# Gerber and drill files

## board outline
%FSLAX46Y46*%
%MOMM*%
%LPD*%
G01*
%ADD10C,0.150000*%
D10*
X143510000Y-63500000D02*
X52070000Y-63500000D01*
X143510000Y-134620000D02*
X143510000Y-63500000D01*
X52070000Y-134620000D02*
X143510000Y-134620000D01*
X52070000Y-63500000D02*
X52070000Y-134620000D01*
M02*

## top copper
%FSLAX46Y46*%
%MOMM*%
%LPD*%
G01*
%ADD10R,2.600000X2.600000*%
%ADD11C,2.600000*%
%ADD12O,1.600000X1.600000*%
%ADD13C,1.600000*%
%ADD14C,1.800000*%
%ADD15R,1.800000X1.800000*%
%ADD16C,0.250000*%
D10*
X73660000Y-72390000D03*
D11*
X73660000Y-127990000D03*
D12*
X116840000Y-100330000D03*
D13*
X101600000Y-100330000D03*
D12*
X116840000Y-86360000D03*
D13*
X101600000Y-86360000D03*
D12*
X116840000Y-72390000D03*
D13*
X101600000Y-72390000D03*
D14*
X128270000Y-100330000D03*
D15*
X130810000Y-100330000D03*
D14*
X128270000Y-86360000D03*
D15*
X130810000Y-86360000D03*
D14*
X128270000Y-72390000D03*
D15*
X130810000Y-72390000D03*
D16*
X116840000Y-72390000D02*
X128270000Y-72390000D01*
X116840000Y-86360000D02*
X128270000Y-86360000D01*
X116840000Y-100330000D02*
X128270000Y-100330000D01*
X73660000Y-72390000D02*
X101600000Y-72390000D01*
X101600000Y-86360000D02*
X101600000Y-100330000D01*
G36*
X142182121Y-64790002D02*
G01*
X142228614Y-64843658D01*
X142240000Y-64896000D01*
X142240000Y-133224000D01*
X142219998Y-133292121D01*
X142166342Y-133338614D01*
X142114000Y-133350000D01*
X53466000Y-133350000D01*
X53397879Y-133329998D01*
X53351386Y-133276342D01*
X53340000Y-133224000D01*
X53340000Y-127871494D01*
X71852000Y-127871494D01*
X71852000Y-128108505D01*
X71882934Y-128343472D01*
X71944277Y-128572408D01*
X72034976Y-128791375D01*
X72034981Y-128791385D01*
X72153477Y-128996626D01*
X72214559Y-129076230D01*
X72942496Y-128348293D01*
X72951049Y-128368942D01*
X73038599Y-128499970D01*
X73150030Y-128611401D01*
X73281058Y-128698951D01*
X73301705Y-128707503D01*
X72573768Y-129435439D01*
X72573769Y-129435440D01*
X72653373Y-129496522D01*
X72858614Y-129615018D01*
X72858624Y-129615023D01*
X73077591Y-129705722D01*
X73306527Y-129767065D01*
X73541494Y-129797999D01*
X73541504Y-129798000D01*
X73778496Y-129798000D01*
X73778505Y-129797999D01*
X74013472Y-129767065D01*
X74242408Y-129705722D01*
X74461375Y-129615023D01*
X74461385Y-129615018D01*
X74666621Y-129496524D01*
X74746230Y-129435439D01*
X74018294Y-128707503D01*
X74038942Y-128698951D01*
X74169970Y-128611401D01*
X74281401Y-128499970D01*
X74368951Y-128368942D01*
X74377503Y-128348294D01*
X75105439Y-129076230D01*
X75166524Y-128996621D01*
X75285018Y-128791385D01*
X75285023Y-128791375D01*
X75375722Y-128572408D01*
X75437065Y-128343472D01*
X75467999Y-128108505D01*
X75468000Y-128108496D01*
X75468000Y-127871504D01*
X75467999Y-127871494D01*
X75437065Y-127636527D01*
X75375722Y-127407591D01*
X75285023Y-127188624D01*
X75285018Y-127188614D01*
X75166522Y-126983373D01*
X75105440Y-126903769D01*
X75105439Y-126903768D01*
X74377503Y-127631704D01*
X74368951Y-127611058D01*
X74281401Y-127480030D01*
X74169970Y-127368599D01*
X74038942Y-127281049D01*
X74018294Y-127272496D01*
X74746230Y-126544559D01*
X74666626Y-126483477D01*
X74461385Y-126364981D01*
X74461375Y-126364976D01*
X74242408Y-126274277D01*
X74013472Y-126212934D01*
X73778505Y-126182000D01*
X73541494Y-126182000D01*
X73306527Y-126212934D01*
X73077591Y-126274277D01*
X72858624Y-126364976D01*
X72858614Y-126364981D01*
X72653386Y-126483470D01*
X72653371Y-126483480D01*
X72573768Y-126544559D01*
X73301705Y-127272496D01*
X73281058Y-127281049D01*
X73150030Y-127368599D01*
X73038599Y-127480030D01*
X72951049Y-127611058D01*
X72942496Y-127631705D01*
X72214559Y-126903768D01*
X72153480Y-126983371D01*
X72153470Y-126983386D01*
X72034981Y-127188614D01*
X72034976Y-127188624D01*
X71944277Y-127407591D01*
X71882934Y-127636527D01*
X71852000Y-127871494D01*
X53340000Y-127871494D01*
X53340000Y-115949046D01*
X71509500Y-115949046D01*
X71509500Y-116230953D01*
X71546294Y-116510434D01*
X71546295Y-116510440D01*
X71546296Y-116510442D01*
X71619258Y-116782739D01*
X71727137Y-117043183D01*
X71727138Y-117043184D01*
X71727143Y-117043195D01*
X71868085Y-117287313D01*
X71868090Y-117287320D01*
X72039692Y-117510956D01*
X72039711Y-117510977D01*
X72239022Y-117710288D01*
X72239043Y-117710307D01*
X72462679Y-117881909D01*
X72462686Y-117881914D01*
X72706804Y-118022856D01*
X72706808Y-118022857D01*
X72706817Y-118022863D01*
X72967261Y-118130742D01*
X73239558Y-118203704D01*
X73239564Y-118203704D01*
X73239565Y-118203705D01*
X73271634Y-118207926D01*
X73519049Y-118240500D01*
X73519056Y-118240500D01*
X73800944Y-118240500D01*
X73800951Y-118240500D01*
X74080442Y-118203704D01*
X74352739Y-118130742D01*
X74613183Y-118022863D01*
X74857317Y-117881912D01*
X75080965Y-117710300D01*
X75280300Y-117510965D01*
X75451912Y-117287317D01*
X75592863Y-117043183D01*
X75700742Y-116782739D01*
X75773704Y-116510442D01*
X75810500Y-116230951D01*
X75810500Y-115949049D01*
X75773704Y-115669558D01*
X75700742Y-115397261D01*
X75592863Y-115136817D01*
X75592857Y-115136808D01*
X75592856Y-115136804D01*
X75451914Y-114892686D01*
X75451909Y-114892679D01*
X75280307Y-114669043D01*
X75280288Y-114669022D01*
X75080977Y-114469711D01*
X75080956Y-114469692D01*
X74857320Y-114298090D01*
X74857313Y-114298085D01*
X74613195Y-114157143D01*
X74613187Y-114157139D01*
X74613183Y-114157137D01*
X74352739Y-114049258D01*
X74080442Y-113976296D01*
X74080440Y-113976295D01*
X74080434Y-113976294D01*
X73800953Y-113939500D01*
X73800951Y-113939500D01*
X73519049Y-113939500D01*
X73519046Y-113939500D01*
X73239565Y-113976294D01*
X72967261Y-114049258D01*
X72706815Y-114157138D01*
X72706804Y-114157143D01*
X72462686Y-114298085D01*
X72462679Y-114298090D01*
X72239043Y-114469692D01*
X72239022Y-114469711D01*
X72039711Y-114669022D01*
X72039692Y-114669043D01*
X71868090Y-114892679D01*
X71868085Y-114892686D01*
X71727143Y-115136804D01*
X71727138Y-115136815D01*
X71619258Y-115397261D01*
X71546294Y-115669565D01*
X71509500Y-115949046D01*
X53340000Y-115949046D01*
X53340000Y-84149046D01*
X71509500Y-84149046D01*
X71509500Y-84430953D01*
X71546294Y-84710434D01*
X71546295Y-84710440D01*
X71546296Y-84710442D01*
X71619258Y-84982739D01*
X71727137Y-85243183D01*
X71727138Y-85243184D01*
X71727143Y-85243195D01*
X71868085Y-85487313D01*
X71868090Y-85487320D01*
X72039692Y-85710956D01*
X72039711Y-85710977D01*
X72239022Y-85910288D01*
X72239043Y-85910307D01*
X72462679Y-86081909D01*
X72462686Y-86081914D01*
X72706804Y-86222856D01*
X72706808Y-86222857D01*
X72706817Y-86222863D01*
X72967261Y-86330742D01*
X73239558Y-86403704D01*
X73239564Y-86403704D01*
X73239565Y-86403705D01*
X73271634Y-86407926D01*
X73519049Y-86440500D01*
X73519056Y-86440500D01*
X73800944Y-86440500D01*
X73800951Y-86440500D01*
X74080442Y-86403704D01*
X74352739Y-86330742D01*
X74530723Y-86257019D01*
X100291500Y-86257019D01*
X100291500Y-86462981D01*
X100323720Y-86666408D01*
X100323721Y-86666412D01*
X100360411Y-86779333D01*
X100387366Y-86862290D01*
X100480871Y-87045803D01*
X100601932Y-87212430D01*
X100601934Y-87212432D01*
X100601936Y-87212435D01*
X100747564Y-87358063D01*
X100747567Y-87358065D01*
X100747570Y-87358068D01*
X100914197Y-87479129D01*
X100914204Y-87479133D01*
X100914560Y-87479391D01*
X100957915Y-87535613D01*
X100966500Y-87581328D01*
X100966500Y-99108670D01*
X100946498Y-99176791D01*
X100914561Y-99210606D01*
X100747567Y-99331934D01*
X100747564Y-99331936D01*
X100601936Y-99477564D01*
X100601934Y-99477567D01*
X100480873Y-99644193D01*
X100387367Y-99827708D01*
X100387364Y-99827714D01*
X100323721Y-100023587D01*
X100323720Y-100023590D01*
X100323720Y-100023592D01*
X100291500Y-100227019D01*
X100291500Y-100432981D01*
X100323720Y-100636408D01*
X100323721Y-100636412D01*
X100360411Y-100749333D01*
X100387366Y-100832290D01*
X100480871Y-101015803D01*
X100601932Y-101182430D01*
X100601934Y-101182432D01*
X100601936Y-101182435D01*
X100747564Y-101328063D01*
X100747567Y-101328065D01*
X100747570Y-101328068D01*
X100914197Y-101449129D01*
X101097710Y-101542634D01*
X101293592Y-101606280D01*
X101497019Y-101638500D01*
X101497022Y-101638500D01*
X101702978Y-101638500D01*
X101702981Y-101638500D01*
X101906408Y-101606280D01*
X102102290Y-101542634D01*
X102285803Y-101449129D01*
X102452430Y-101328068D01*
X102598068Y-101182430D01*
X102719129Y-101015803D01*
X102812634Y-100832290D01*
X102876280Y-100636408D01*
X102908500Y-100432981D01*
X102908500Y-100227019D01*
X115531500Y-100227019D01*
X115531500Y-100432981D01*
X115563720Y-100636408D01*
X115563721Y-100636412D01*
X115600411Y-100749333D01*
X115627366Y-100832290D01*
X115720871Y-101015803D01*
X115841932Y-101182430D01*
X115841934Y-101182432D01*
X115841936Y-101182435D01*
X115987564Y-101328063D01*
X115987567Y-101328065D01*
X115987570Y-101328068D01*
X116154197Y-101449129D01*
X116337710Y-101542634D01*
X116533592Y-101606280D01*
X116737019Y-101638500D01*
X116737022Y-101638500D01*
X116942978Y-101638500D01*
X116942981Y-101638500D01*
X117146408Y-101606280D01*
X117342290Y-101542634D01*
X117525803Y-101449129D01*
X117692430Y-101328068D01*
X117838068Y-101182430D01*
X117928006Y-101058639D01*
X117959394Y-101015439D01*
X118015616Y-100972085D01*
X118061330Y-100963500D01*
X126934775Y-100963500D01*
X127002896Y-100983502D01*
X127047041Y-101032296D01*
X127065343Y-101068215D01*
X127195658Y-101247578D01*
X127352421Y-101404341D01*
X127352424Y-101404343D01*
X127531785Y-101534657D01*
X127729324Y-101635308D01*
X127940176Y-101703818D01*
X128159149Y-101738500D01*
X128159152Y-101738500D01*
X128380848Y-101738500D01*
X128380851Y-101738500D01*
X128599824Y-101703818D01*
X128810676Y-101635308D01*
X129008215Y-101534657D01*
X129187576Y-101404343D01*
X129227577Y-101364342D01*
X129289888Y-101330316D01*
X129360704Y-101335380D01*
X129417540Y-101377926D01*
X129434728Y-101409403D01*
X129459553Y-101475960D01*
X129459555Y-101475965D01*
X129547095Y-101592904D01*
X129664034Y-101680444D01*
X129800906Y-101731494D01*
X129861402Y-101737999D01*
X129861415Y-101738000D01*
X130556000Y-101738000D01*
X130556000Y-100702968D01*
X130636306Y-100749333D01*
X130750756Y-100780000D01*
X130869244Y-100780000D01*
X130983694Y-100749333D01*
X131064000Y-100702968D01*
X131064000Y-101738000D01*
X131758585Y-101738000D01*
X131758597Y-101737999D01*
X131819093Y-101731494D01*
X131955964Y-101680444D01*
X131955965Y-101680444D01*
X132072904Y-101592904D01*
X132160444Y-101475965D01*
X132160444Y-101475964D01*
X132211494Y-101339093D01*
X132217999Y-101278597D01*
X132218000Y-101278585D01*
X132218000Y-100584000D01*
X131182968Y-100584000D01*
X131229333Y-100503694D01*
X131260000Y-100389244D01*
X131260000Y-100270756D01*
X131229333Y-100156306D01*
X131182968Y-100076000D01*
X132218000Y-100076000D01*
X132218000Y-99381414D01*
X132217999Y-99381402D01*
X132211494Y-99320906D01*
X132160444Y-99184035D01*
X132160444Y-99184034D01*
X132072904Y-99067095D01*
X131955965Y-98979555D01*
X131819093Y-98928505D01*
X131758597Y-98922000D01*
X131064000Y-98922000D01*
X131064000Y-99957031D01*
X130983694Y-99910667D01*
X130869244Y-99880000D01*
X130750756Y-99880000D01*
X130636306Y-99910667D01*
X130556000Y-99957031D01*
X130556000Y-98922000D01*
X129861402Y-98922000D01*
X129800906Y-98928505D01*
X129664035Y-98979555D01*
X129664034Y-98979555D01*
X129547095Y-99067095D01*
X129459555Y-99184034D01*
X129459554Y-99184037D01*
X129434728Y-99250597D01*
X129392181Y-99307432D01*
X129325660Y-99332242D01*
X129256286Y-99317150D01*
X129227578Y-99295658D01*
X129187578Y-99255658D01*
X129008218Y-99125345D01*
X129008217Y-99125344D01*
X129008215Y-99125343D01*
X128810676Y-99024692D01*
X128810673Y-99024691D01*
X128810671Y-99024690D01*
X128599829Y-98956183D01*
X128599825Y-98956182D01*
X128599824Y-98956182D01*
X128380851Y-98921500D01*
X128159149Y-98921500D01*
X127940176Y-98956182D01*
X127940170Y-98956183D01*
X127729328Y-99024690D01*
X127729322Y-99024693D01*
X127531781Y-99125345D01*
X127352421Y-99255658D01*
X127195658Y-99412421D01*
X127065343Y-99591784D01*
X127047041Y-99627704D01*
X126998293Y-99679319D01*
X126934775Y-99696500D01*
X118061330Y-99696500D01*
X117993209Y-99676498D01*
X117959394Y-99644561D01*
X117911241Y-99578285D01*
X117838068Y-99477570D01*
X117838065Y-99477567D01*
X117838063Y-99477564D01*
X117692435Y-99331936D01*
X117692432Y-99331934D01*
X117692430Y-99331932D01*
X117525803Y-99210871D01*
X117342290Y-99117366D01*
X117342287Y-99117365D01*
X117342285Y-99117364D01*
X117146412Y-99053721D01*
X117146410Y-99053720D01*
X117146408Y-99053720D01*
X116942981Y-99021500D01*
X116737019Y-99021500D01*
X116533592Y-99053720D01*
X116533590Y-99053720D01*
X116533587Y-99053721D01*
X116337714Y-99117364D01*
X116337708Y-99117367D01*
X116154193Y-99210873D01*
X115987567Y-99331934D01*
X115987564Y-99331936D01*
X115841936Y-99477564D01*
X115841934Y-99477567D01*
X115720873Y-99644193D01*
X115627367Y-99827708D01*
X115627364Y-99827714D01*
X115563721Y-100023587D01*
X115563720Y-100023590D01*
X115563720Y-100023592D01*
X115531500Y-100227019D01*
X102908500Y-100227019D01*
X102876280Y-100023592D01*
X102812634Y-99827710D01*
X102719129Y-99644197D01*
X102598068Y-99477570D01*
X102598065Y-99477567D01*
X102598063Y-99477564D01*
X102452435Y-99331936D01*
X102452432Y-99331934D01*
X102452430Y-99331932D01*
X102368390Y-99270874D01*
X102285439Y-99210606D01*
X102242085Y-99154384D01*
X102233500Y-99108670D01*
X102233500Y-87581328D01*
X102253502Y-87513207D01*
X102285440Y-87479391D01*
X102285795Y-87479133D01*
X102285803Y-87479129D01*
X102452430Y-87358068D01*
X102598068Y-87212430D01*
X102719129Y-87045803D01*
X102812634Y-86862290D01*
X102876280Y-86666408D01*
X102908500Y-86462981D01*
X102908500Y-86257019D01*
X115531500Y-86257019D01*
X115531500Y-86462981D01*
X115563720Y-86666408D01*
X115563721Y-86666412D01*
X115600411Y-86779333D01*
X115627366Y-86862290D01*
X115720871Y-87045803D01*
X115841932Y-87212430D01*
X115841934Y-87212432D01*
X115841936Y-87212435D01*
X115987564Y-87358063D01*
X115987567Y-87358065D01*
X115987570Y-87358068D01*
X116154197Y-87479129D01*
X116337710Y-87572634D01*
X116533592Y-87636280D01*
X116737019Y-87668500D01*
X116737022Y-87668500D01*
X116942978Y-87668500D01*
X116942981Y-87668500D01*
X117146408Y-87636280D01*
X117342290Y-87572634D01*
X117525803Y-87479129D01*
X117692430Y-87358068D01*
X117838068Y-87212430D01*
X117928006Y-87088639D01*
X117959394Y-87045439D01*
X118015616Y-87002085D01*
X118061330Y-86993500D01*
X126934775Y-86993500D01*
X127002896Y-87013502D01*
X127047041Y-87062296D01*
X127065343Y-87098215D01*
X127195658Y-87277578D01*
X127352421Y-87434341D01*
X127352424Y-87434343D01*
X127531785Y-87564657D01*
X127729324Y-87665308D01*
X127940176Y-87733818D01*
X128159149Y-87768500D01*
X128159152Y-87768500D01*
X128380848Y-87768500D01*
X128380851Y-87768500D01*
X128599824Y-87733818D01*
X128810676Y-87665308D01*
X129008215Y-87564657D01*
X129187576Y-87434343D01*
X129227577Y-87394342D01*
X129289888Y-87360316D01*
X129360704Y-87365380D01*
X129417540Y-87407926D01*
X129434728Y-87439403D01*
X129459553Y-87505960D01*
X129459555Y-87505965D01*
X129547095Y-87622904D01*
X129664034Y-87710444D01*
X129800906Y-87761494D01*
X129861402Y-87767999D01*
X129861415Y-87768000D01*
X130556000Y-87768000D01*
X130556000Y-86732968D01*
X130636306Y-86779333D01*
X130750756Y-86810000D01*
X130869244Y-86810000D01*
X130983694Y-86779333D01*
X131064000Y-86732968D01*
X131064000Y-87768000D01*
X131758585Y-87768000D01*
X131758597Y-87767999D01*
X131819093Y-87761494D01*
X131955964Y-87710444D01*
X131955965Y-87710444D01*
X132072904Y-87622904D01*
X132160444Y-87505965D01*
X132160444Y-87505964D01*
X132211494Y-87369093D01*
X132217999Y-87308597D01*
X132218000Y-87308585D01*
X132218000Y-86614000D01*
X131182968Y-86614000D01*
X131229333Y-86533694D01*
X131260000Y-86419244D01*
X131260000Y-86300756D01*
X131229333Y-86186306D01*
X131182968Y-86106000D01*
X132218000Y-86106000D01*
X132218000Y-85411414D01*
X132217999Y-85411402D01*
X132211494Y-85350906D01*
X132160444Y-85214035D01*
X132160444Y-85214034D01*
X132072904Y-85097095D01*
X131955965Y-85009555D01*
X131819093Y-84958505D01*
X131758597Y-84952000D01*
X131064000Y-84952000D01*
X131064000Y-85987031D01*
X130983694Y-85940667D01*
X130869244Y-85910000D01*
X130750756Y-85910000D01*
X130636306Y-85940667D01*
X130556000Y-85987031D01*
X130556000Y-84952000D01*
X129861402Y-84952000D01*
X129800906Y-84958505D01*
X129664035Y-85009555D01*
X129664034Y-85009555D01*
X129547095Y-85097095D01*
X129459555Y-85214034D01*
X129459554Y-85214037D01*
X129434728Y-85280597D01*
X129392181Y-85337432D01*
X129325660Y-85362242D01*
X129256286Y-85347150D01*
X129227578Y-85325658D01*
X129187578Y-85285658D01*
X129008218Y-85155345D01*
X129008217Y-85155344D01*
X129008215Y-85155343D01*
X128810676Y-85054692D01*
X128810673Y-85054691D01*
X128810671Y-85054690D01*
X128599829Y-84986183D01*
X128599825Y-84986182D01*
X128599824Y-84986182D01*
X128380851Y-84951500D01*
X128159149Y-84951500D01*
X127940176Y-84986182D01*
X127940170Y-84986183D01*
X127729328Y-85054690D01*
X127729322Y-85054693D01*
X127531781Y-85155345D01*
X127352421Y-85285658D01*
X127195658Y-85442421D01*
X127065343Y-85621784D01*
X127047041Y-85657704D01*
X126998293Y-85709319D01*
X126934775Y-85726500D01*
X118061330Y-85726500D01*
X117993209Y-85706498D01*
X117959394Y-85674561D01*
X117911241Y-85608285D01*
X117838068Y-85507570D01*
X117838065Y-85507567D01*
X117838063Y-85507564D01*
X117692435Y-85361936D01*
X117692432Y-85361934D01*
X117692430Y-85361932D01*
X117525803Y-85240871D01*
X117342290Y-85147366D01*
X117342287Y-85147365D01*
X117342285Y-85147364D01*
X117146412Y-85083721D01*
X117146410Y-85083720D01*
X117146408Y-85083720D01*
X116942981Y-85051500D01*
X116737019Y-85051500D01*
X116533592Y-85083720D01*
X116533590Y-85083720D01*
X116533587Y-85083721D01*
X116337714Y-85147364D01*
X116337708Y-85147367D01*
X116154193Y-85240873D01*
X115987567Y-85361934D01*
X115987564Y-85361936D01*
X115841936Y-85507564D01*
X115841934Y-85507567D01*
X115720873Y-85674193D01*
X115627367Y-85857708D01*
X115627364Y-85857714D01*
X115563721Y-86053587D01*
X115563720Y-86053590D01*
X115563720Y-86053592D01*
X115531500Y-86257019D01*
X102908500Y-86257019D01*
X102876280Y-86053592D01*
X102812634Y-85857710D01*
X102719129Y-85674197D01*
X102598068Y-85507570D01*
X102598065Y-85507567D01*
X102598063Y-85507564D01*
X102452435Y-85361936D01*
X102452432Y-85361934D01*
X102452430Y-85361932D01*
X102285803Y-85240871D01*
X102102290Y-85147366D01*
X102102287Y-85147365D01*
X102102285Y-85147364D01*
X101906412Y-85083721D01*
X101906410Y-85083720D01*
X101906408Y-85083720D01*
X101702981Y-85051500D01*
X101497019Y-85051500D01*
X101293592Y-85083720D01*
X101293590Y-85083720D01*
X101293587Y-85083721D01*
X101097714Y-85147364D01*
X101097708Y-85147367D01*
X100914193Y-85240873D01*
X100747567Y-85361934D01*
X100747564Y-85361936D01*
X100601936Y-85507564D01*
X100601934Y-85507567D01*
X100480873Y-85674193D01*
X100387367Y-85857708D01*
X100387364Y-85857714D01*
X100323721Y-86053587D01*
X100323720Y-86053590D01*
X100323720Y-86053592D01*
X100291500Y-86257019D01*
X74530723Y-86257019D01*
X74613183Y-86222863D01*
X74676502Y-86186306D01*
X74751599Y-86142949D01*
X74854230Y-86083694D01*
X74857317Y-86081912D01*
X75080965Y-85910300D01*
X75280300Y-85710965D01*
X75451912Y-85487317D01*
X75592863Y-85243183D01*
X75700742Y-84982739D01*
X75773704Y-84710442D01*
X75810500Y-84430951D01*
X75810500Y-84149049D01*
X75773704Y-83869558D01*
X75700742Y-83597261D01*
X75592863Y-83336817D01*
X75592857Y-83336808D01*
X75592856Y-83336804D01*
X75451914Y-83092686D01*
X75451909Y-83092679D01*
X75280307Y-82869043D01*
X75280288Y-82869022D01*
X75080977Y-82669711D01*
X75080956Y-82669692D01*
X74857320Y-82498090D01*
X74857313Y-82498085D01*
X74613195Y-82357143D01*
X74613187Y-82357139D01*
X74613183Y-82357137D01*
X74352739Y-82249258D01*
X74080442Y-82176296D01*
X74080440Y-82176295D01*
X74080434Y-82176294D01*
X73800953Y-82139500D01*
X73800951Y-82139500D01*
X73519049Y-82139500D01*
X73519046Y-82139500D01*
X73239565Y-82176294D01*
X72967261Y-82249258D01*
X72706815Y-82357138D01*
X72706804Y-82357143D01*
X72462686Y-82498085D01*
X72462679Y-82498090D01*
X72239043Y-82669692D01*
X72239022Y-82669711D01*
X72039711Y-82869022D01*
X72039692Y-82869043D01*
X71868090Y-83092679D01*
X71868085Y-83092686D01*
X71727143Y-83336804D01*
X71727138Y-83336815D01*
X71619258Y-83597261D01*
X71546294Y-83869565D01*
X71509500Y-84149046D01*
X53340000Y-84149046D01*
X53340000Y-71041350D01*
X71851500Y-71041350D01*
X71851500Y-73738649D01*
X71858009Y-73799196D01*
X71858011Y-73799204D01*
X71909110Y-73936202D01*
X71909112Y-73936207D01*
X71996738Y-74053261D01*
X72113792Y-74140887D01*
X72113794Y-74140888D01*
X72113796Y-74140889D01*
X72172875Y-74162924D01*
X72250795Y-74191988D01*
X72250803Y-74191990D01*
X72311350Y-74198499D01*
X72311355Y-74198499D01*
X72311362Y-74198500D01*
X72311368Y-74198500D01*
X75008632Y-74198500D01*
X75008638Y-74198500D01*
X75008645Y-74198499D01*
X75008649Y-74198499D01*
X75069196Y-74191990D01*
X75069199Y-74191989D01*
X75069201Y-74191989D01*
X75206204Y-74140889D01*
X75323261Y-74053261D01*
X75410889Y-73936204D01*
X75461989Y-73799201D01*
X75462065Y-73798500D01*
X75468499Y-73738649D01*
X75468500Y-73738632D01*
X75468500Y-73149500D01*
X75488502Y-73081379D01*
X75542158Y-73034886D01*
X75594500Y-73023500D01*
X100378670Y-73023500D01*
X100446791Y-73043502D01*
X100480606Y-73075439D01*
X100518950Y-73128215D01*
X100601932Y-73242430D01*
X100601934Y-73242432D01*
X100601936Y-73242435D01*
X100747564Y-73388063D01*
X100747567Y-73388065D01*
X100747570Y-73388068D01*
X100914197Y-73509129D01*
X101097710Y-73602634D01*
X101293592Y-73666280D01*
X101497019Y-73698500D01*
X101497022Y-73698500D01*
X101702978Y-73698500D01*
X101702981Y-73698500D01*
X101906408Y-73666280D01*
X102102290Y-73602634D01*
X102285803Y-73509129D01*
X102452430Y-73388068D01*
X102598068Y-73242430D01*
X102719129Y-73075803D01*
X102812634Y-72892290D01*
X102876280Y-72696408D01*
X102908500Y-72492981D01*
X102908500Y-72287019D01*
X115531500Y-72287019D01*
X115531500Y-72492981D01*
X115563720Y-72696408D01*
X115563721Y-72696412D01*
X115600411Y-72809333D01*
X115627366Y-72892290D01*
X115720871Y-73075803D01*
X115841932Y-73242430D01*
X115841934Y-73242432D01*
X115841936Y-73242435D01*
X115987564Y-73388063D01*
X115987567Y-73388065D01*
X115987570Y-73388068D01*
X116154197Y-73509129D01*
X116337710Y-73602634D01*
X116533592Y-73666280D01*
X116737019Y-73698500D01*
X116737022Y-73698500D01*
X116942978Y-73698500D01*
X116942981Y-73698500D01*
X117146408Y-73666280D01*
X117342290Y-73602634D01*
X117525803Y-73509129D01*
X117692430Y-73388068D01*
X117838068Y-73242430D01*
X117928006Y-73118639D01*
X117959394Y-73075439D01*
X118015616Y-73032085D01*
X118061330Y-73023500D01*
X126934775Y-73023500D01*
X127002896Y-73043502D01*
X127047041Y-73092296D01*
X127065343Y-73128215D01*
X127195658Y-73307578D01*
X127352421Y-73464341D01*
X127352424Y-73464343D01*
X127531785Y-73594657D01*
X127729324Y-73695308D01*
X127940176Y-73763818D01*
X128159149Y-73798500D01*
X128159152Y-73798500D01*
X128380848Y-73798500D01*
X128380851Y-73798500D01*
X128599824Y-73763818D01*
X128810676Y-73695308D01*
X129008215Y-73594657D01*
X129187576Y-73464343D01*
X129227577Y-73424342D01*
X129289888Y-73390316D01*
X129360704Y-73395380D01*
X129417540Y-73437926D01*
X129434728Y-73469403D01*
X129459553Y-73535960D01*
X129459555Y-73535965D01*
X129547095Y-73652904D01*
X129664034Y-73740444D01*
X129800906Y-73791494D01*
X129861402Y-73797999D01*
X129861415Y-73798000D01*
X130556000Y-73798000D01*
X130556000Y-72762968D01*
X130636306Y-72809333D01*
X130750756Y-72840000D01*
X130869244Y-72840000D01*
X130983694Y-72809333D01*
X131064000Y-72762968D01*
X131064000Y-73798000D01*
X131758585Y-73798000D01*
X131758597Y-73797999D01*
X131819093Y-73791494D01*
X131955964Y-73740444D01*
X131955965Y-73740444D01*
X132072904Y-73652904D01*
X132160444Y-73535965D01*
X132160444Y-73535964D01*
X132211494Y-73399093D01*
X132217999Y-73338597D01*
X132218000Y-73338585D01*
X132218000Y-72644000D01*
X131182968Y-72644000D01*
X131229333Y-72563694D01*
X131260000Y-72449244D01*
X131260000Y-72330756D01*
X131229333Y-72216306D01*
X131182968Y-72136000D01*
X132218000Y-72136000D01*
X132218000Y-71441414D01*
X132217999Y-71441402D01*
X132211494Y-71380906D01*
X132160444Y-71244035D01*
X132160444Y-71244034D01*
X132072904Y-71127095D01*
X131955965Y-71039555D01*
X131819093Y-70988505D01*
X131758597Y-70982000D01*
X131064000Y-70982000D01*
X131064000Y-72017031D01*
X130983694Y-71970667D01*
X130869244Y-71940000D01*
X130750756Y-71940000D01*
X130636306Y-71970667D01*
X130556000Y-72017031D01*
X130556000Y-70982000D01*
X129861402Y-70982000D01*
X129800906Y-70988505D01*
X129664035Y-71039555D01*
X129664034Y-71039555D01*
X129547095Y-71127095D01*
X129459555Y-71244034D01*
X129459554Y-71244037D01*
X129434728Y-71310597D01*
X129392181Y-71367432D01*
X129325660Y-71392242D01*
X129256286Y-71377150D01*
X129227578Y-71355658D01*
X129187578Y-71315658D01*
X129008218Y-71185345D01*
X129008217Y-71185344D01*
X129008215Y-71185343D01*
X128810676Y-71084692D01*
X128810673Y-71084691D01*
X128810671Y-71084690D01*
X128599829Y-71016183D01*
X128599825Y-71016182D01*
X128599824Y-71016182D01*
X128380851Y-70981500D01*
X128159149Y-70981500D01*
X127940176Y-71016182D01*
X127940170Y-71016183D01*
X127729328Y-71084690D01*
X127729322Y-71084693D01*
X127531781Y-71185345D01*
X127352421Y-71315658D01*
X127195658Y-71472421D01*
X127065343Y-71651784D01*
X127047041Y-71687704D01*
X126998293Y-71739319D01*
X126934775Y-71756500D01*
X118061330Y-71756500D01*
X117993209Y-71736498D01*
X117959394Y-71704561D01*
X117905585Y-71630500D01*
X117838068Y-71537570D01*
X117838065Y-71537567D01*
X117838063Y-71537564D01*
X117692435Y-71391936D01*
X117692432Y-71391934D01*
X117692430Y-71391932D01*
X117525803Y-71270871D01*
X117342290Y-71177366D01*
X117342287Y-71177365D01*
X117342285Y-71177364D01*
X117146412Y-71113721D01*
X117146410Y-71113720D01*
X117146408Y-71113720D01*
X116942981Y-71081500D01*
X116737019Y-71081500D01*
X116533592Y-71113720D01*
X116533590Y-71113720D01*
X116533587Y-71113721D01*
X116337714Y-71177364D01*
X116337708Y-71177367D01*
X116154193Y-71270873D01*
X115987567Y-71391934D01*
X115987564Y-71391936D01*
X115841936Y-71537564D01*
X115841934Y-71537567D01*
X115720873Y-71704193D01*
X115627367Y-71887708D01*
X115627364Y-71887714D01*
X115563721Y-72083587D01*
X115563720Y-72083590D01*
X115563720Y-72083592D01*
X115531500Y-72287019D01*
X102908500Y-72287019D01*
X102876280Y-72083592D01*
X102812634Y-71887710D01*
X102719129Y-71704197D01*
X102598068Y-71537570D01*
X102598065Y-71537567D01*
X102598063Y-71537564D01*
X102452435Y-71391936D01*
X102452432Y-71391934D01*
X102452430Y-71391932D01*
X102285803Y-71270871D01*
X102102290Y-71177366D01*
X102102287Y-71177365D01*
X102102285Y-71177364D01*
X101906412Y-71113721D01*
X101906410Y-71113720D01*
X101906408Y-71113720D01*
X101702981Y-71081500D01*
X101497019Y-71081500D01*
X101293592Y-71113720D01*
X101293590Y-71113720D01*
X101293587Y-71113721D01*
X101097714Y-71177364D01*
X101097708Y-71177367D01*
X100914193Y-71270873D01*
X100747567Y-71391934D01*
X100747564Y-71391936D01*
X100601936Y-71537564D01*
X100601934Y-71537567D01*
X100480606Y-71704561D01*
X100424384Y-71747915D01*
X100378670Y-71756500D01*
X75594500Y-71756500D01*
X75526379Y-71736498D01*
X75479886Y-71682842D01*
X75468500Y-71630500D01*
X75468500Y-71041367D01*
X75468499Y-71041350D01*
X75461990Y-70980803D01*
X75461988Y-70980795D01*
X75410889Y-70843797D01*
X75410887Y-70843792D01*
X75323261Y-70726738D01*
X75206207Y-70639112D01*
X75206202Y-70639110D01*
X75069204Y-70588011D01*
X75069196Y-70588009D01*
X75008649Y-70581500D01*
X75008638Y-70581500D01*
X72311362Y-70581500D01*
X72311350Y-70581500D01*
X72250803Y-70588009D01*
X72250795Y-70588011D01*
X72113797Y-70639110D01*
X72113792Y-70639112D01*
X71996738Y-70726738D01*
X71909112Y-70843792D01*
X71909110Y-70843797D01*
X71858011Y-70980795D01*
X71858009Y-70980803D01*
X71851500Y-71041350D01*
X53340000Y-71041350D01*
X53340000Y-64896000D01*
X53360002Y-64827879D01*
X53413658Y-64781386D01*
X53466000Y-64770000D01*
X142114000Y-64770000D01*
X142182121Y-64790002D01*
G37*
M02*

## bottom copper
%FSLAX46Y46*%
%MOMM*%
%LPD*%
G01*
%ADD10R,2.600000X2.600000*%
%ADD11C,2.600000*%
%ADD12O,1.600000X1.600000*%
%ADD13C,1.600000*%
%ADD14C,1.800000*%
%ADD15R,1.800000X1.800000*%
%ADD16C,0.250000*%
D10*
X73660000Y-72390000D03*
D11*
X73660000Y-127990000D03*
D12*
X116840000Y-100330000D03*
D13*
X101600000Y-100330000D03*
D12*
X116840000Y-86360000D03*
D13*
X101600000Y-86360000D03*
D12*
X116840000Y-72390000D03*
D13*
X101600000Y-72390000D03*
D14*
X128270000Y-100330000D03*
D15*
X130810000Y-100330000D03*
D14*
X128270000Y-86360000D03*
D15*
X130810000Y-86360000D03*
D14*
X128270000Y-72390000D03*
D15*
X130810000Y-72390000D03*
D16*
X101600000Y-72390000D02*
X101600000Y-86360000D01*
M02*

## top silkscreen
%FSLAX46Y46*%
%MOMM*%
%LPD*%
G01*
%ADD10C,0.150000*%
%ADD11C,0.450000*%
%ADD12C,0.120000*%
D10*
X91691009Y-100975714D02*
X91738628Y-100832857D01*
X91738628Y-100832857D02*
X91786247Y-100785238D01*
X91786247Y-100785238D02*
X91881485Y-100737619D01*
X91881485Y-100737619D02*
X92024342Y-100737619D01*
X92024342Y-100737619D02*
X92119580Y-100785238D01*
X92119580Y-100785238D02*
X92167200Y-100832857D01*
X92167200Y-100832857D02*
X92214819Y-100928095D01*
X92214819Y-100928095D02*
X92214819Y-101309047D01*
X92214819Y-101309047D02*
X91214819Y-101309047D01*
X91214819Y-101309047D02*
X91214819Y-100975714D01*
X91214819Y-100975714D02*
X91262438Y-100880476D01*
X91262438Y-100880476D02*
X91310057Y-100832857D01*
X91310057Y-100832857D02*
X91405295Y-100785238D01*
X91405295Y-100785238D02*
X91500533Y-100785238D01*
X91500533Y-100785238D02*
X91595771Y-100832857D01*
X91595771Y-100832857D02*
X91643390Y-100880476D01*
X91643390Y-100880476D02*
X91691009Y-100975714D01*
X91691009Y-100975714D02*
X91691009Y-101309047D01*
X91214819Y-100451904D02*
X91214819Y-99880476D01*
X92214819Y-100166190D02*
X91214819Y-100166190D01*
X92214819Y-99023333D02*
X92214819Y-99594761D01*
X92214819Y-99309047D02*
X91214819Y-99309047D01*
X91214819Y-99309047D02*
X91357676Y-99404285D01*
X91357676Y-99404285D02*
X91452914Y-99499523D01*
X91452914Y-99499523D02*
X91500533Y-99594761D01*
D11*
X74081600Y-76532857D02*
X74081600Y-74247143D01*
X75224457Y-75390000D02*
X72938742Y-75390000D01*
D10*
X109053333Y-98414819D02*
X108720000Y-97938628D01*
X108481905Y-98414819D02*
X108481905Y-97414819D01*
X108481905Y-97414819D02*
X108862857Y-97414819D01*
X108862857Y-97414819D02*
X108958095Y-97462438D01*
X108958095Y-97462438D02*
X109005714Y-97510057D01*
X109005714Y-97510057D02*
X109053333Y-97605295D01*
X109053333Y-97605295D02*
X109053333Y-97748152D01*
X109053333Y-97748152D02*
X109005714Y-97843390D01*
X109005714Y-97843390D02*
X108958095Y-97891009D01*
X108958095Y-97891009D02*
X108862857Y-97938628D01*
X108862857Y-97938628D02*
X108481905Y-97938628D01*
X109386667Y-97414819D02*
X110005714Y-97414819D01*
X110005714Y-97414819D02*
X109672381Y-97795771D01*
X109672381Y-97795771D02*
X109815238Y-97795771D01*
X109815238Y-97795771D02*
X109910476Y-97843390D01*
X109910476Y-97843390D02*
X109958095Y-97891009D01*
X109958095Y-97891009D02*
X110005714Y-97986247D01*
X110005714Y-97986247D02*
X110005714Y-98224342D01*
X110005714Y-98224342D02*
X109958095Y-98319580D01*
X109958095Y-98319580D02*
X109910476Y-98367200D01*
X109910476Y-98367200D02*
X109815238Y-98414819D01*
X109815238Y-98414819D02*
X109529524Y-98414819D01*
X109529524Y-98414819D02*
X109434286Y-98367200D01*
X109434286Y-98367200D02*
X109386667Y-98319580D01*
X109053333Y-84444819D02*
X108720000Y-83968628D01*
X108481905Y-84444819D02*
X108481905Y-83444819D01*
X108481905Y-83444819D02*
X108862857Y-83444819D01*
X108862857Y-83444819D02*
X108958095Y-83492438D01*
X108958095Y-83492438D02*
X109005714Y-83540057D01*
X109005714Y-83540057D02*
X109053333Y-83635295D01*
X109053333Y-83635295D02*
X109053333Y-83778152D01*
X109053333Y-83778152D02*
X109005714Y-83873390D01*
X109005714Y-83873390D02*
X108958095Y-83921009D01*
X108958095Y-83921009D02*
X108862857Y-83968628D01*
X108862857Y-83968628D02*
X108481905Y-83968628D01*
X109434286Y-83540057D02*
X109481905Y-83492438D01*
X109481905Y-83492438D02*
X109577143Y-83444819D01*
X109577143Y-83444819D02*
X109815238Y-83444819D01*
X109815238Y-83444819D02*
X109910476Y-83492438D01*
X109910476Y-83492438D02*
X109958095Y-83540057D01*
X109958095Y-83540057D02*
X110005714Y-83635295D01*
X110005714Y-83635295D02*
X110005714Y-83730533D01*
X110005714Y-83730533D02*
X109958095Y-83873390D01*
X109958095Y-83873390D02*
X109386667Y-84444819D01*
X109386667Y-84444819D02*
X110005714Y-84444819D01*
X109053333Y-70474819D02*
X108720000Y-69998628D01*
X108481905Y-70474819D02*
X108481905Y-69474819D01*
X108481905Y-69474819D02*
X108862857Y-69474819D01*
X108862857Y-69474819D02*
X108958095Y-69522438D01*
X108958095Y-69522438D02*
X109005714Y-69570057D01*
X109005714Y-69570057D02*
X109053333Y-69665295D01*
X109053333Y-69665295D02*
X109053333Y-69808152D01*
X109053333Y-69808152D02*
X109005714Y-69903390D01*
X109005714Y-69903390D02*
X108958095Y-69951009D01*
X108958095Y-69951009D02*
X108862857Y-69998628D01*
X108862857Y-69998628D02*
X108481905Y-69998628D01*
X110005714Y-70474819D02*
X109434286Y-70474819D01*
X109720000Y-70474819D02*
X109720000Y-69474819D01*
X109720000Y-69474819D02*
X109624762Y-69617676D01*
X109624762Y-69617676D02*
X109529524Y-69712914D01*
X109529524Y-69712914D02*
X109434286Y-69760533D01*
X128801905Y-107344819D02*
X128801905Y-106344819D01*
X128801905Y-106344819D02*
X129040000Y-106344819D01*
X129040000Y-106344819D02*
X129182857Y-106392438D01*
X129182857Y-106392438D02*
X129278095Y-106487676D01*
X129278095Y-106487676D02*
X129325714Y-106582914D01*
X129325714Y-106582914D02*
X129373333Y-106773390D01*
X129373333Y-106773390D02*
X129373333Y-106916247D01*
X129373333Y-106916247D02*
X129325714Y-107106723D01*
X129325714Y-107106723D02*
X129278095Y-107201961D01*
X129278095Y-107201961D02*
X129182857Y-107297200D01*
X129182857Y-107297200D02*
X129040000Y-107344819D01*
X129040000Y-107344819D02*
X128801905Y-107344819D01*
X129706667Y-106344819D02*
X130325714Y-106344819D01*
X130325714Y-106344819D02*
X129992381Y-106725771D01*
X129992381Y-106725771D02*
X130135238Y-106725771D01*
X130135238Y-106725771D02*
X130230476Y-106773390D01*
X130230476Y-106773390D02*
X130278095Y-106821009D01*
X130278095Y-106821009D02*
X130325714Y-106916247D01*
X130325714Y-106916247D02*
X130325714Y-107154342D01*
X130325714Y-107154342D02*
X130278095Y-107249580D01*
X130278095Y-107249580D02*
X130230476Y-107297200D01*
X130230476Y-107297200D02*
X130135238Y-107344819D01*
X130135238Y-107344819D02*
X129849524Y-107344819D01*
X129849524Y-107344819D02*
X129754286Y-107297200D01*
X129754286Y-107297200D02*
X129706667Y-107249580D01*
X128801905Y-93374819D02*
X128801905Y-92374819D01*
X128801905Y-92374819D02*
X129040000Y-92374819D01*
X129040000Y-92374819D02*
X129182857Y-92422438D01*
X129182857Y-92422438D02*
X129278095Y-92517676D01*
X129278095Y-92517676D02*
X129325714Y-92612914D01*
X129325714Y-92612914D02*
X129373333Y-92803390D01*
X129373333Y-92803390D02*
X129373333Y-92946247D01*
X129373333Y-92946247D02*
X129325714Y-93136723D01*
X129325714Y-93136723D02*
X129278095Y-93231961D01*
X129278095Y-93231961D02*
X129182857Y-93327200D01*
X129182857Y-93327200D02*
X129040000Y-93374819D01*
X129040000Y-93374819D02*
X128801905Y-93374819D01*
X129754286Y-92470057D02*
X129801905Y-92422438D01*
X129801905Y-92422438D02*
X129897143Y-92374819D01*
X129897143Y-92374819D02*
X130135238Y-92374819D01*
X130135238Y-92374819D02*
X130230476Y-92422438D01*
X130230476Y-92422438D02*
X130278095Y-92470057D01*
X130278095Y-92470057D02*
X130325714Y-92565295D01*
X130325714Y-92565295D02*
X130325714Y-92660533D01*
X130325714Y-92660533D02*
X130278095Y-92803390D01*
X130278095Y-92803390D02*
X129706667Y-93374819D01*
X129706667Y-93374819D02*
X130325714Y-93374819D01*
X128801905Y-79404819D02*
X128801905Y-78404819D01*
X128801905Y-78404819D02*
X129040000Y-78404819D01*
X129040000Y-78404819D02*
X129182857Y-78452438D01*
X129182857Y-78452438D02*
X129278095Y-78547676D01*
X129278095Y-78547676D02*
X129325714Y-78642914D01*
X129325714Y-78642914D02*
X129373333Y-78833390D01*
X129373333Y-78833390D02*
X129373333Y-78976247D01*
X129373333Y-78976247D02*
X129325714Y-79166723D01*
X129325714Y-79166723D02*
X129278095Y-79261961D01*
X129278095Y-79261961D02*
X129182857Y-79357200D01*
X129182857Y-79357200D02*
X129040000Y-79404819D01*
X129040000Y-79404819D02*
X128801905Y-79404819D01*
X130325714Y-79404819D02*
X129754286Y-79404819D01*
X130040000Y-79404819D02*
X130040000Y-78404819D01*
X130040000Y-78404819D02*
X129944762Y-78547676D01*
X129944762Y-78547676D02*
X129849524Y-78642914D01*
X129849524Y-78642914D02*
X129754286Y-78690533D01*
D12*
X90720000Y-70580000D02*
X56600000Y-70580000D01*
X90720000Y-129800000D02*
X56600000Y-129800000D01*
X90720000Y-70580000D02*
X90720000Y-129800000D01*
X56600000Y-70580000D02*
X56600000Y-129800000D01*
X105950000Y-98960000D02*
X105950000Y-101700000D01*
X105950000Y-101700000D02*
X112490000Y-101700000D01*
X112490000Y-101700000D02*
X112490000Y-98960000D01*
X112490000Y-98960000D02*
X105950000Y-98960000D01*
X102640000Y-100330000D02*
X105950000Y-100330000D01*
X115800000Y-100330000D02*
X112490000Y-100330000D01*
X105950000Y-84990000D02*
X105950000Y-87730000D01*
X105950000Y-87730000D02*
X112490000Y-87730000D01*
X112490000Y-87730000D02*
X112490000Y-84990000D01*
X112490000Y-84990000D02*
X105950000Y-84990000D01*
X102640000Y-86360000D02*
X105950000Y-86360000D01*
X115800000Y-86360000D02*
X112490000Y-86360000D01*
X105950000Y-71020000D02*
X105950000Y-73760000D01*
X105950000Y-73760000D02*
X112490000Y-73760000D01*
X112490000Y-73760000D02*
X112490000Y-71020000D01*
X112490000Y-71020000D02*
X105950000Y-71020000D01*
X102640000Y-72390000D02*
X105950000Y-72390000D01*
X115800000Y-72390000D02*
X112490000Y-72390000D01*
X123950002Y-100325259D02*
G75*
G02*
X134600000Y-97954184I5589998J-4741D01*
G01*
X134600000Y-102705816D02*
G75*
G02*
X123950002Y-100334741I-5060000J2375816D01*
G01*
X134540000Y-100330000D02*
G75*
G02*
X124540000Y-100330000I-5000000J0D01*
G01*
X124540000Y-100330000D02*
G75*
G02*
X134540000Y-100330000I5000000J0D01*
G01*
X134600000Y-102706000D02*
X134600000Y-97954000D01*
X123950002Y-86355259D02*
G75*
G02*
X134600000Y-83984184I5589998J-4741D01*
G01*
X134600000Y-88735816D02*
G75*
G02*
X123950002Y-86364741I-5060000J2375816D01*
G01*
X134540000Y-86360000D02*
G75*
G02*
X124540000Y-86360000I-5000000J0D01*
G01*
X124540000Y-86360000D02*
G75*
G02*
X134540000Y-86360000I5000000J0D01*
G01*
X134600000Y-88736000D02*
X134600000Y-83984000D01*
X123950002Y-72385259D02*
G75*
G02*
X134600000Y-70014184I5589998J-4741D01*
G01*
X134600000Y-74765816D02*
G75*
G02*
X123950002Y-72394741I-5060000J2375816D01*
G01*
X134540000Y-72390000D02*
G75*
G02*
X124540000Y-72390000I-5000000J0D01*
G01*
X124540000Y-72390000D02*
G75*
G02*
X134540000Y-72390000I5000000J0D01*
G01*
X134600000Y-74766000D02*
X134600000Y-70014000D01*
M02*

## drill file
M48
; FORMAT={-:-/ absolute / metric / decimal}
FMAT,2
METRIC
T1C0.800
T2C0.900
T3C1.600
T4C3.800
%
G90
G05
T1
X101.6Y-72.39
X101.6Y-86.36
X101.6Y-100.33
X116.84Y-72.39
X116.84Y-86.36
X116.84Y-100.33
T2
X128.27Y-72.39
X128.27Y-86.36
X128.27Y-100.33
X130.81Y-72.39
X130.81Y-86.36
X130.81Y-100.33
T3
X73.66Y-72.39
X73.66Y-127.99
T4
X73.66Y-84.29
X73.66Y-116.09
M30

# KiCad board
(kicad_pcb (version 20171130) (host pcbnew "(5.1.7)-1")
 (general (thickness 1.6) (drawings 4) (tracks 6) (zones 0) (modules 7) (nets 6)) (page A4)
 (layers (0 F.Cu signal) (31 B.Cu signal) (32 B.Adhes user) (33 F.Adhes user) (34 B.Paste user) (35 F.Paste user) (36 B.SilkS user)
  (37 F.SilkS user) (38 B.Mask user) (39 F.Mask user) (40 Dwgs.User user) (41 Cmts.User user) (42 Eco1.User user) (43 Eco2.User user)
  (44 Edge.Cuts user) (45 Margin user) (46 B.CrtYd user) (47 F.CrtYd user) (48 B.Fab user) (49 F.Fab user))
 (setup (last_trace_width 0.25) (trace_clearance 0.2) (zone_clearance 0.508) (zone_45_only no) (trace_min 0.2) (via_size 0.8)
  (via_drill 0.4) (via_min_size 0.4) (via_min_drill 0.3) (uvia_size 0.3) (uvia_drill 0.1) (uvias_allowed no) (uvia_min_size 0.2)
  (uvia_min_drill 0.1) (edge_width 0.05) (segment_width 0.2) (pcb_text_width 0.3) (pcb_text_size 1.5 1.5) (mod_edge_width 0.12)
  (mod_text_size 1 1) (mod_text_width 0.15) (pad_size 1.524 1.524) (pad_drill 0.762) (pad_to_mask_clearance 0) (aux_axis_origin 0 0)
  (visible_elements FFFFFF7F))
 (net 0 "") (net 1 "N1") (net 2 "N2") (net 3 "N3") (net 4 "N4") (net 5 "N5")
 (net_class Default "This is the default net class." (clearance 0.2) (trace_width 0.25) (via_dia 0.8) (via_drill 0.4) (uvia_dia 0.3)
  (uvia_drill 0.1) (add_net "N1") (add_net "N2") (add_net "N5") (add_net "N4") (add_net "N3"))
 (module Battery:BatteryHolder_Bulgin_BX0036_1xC (layer F.Cu) (at 73.66 72.39 270)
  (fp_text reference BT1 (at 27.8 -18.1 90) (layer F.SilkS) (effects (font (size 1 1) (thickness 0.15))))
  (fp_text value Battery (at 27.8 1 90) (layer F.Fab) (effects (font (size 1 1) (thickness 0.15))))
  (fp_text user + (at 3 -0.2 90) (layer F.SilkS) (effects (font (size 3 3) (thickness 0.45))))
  (fp_line (start -1.81 -17.06) (end -1.81 17.06) (layer F.SilkS) (width 0.12))
  (fp_line (start 57.41 -17.06) (end 57.41 17.06) (layer F.SilkS) (width 0.12))
  (fp_line (start -1.81 -17.06) (end 57.41 -17.06) (layer F.SilkS) (width 0.12))
  (fp_line (start -1.81 17.06) (end 57.41 17.06) (layer F.SilkS) (width 0.12))
  (pad "" np_thru_hole circle (at 43.7 0 270) (size 3.8 3.8) (drill 3.8) (layers *.Cu *.Mask))
  (pad "" np_thru_hole circle (at 11.9 0 270) (size 3.8 3.8) (drill 3.8) (layers *.Cu *.Mask))
  (pad 1 thru_hole rect (at 0 0 270) (size 2.6 2.6) (drill 1.6) (layers *.Cu *.Mask) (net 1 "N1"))
  (pad 2 thru_hole circle (at 55.6 0 270) (size 2.6 2.6) (drill 1.6) (layers *.Cu *.Mask) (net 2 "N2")))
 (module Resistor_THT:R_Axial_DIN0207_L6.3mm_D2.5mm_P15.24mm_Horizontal (layer F.Cu) (at 101.6 100.33)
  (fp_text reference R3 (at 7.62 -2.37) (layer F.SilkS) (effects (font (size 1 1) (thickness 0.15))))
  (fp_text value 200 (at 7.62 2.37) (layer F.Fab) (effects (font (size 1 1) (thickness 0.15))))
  (fp_line (start 4.35 -1.37) (end 4.35 1.37) (layer F.SilkS) (width 0.12))
  (fp_line (start 4.35 1.37) (end 10.89 1.37) (layer F.SilkS) (width 0.12))
  (fp_line (start 10.89 1.37) (end 10.89 -1.37) (layer F.SilkS) (width 0.12))
  (fp_line (start 10.89 -1.37) (end 4.35 -1.37) (layer F.SilkS) (width 0.12))
  (fp_line (start 1.04 0) (end 4.35 0) (layer F.SilkS) (width 0.12))
  (fp_line (start 14.2 0) (end 10.89 0) (layer F.SilkS) (width 0.12))
  (pad 2 thru_hole oval (at 15.24 0) (size 1.6 1.6) (drill 0.8) (layers *.Cu *.Mask) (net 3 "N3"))
  (pad 1 thru_hole circle (at 0 0) (size 1.6 1.6) (drill 0.8) (layers *.Cu *.Mask) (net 1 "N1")))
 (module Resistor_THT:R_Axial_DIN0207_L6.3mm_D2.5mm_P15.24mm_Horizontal (layer F.Cu) (at 101.6 86.36)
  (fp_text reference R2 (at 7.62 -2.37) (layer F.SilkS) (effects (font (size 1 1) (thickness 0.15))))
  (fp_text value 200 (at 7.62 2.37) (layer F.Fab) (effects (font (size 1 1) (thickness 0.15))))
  (fp_line (start 4.35 -1.37) (end 4.35 1.37) (layer F.SilkS) (width 0.12))
  (fp_line (start 4.35 1.37) (end 10.89 1.37) (layer F.SilkS) (width 0.12))
  (fp_line (start 10.89 1.37) (end 10.89 -1.37) (layer F.SilkS) (width 0.12))
  (fp_line (start 10.89 -1.37) (end 4.35 -1.37) (layer F.SilkS) (width 0.12))
  (fp_line (start 1.04 0) (end 4.35 0) (layer F.SilkS) (width 0.12))
  (fp_line (start 14.2 0) (end 10.89 0) (layer F.SilkS) (width 0.12))
  (pad 2 thru_hole oval (at 15.24 0) (size 1.6 1.6) (drill 0.8) (layers *.Cu *.Mask) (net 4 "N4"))
  (pad 1 thru_hole circle (at 0 0) (size 1.6 1.6) (drill 0.8) (layers *.Cu *.Mask) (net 1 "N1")))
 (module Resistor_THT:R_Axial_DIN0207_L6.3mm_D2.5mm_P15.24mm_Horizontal (layer F.Cu) (at 101.6 72.39)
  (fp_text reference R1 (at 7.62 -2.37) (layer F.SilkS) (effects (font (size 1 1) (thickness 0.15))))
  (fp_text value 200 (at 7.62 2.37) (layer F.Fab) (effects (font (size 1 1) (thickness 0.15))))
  (fp_line (start 4.35 -1.37) (end 4.35 1.37) (layer F.SilkS) (width 0.12))
  (fp_line (start 4.35 1.37) (end 10.89 1.37) (layer F.SilkS) (width 0.12))
  (fp_line (start 10.89 1.37) (end 10.89 -1.37) (layer F.SilkS) (width 0.12))
  (fp_line (start 10.89 -1.37) (end 4.35 -1.37) (layer F.SilkS) (width 0.12))
  (fp_line (start 1.04 0) (end 4.35 0) (layer F.SilkS) (width 0.12))
  (fp_line (start 14.2 0) (end 10.89 0) (layer F.SilkS) (width 0.12))
  (pad 2 thru_hole oval (at 15.24 0) (size 1.6 1.6) (drill 0.8) (layers *.Cu *.Mask) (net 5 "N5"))
  (pad 1 thru_hole circle (at 0 0) (size 1.6 1.6) (drill 0.8) (layers *.Cu *.Mask) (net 1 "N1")))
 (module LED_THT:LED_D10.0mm (layer F.Cu) (at 130.81 100.33 180)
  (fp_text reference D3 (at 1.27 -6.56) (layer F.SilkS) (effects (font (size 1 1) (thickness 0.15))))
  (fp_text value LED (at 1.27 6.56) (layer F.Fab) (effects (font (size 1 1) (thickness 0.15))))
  (fp_arc (start 1.27 0) (end -3.79 2.375816) (angle -154.8) (layer F.SilkS) (width 0.12))
  (fp_arc (start 1.27 0) (end -3.79 -2.375816) (angle 154.8) (layer F.SilkS) (width 0.12))
  (fp_circle (center 1.27 0) (end 6.27 0) (layer F.SilkS) (width 0.12))
  (fp_line (start -3.79 -2.376) (end -3.79 2.376) (layer F.SilkS) (width 0.12))
  (pad 2 thru_hole circle (at 2.54 0 180) (size 1.8 1.8) (drill 0.9) (layers *.Cu *.Mask) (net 3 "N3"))
  (pad 1 thru_hole rect (at 0 0 180) (size 1.8 1.8) (drill 0.9) (layers *.Cu *.Mask) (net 2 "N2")))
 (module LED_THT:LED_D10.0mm (layer F.Cu) (at 130.81 86.36 180)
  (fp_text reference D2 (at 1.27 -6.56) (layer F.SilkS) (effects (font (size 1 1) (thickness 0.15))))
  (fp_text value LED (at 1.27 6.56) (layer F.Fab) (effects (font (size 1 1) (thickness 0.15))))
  (fp_arc (start 1.27 0) (end -3.79 2.375816) (angle -154.8) (layer F.SilkS) (width 0.12))
  (fp_arc (start 1.27 0) (end -3.79 -2.375816) (angle 154.8) (layer F.SilkS) (width 0.12))
  (fp_circle (center 1.27 0) (end 6.27 0) (layer F.SilkS) (width 0.12))
  (fp_line (start -3.79 -2.376) (end -3.79 2.376) (layer F.SilkS) (width 0.12))
  (pad 2 thru_hole circle (at 2.54 0 180) (size 1.8 1.8) (drill 0.9) (layers *.Cu *.Mask) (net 4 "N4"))
  (pad 1 thru_hole rect (at 0 0 180) (size 1.8 1.8) (drill 0.9) (layers *.Cu *.Mask) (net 2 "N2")))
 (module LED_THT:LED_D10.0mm (layer F.Cu) (at 130.81 72.39 180)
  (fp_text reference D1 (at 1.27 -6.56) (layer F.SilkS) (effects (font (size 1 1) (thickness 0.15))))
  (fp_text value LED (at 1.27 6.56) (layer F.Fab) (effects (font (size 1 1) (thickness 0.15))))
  (fp_arc (start 1.27 0) (end -3.79 2.375816) (angle -154.8) (layer F.SilkS) (width 0.12))
  (fp_arc (start 1.27 0) (end -3.79 -2.375816) (angle 154.8) (layer F.SilkS) (width 0.12))
  (fp_circle (center 1.27 0) (end 6.27 0) (layer F.SilkS) (width 0.12))
  (fp_line (start -3.79 -2.376) (end -3.79 2.376) (layer F.SilkS) (width 0.12))
  (pad 2 thru_hole circle (at 2.54 0 180) (size 1.8 1.8) (drill 0.9) (layers *.Cu *.Mask) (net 5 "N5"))
  (pad 1 thru_hole rect (at 0 0 180) (size 1.8 1.8) (drill 0.9) (layers *.Cu *.Mask) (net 2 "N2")))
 (gr_line (start 143.51 63.5) (end 52.07 63.5) (layer Edge.Cuts) (width 0.15))
 (gr_line (start 143.51 134.62) (end 143.51 63.5) (layer Edge.Cuts) (width 0.15))
 (gr_line (start 52.07 134.62) (end 143.51 134.62) (layer Edge.Cuts) (width 0.15))
 (gr_line (start 52.07 63.5) (end 52.07 134.62) (layer Edge.Cuts) (width 0.15))
 (segment (start 116.84 72.39) (end 128.27 72.39) (width 0.25) (layer F.Cu) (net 5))
 (segment (start 116.84 86.36) (end 128.27 86.36) (width 0.25) (layer F.Cu) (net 4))
 (segment (start 116.84 100.33) (end 128.27 100.33) (width 0.25) (layer F.Cu) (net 3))
 (segment (start 73.66 72.39) (end 101.6 72.39) (width 0.25) (layer F.Cu) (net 1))
 (segment (start 101.6 72.39) (end 101.6 86.36) (width 0.25) (layer B.Cu) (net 1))
 (segment (start 101.6 86.36) (end 101.6 100.33) (width 0.25) (layer F.Cu) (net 1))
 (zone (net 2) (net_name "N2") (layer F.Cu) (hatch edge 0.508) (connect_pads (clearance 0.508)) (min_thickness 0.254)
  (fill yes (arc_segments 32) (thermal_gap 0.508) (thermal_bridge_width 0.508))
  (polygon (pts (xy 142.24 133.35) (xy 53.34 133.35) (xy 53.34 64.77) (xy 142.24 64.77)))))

